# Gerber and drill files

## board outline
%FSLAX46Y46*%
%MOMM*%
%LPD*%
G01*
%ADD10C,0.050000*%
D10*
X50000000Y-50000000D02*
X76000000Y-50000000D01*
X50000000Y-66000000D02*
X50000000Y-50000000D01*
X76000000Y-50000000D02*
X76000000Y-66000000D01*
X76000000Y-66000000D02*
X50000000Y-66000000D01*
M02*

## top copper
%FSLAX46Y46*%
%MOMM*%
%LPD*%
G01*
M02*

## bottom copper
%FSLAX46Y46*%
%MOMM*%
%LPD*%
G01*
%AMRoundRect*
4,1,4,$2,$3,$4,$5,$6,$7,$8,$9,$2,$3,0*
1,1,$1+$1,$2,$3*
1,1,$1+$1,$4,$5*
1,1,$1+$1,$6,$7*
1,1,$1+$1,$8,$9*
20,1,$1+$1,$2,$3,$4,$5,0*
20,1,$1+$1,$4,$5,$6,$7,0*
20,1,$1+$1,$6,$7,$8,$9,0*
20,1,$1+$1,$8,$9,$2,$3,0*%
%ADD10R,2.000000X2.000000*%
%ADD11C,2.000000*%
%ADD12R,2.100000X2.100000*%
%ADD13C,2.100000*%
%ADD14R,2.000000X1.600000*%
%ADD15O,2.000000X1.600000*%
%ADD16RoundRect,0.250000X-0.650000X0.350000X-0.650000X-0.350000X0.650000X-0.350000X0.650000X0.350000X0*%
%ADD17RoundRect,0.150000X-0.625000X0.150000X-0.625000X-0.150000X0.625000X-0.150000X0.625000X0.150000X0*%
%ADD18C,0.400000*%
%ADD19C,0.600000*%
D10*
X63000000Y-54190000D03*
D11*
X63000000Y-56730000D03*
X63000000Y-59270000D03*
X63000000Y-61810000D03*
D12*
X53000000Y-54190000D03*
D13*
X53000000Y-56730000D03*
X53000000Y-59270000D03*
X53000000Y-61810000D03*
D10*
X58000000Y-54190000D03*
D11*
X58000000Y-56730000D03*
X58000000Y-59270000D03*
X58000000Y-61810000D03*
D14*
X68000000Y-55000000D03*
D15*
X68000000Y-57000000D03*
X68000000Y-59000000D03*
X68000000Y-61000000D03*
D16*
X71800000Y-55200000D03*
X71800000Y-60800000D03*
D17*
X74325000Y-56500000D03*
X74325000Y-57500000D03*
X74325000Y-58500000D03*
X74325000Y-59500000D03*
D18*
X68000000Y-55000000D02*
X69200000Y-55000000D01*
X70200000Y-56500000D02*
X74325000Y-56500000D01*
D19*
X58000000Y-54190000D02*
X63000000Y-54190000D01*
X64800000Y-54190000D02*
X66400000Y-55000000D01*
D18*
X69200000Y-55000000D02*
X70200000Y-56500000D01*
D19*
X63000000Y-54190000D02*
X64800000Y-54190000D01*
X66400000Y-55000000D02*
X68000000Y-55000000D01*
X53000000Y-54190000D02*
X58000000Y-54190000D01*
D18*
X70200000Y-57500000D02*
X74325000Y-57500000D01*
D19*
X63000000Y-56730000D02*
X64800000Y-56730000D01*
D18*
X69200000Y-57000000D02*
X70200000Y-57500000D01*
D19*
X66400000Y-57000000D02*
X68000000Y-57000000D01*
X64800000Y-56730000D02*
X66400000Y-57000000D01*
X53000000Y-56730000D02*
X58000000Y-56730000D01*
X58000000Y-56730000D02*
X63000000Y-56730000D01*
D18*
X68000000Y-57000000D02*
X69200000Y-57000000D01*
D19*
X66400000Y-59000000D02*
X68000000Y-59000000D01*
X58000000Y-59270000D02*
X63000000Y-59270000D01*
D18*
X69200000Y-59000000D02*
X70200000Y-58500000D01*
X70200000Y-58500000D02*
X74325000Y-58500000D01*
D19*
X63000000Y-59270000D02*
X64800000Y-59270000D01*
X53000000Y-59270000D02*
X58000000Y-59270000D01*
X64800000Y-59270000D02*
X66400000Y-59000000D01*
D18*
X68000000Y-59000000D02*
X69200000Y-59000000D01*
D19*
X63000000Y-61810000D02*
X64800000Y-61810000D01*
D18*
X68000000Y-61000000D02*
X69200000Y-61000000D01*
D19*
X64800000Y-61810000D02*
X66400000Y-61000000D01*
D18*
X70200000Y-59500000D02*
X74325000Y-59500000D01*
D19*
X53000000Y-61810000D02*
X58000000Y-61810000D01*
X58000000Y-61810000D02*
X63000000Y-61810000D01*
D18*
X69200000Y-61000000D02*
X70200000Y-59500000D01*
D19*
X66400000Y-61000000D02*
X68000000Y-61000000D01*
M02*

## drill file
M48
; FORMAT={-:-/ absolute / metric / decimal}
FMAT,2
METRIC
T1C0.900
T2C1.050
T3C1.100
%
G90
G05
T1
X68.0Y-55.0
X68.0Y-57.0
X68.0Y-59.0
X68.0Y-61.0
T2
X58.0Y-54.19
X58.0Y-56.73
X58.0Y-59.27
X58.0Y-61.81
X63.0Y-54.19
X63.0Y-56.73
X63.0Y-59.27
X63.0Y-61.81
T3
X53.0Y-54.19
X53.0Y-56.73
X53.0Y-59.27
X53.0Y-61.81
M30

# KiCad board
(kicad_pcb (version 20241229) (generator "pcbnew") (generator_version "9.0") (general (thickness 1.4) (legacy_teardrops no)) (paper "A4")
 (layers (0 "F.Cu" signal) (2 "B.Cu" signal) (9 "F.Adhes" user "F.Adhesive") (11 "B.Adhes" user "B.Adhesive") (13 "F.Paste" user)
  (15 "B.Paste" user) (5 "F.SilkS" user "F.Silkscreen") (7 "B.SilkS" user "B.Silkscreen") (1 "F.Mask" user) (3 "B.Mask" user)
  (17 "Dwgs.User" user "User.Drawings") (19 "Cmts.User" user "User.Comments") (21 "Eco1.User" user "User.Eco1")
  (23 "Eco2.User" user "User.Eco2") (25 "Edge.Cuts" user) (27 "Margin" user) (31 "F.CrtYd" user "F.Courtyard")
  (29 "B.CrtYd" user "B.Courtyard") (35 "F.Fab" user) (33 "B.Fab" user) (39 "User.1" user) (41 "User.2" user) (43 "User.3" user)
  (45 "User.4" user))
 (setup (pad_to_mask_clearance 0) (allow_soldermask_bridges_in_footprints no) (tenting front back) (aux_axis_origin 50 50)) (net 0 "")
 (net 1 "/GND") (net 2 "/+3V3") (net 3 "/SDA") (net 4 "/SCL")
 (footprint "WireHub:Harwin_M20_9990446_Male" (layer "F.Cu") (at 63 54.19)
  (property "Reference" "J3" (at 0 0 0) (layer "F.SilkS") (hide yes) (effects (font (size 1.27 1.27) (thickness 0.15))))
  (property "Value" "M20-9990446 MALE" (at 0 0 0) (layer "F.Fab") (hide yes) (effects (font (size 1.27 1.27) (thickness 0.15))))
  (pad "1" thru_hole rect (at 0 0) (size 2 2) (drill 1.05) (layers "*.Cu" "*.Mask") (remove_unused_layers yes) (keep_end_layers no)
   (zone_layer_connections) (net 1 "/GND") (thermal_bridge_angle 45))
  (pad "2" thru_hole circle (at 0 2.54) (size 2 2) (drill 1.05) (layers "*.Cu" "*.Mask") (remove_unused_layers yes) (keep_end_layers no)
   (zone_layer_connections) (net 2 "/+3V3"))
  (pad "3" thru_hole circle (at 0 5.08) (size 2 2) (drill 1.05) (layers "*.Cu" "*.Mask") (remove_unused_layers yes) (keep_end_layers no)
   (zone_layer_connections) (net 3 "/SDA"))
  (pad "4" thru_hole circle (at 0 7.62) (size 2 2) (drill 1.05) (layers "*.Cu" "*.Mask") (remove_unused_layers yes) (keep_end_layers no)
   (zone_layer_connections) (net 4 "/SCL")))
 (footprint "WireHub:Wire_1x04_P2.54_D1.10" (layer "F.Cu") (at 53 54.19)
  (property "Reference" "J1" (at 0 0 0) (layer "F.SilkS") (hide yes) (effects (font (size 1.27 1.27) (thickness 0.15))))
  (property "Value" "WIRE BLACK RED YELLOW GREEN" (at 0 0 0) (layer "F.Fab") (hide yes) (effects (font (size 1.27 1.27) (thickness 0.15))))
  (pad "1" thru_hole rect (at 0 0) (size 2.1 2.1) (drill 1.1) (layers "*.Cu" "*.Mask") (remove_unused_layers yes) (keep_end_layers no)
   (zone_layer_connections) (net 1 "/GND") (thermal_bridge_angle 45))
  (pad "2" thru_hole circle (at 0 2.54) (size 2.1 2.1) (drill 1.1) (layers "*.Cu" "*.Mask") (remove_unused_layers yes) (keep_end_layers no)
   (zone_layer_connections) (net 2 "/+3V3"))
  (pad "3" thru_hole circle (at 0 5.08) (size 2.1 2.1) (drill 1.1) (layers "*.Cu" "*.Mask") (remove_unused_layers yes) (keep_end_layers no)
   (zone_layer_connections) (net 3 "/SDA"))
  (pad "4" thru_hole circle (at 0 7.62) (size 2.1 2.1) (drill 1.1) (layers "*.Cu" "*.Mask") (remove_unused_layers yes) (keep_end_layers no)
   (zone_layer_connections) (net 4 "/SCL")))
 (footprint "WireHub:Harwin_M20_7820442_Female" (layer "F.Cu") (at 58 54.19)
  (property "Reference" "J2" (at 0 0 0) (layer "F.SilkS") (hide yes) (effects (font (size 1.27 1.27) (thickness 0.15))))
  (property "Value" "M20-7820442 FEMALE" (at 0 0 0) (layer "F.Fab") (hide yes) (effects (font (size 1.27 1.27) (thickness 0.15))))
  (pad "1" thru_hole rect (at 0 0) (size 2 2) (drill 1.05) (layers "*.Cu" "*.Mask") (remove_unused_layers yes) (keep_end_layers no)
   (zone_layer_connections) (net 1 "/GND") (thermal_bridge_angle 45))
  (pad "2" thru_hole circle (at 0 2.54) (size 2 2) (drill 1.05) (layers "*.Cu" "*.Mask") (remove_unused_layers yes) (keep_end_layers no)
   (zone_layer_connections) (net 2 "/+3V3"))
  (pad "3" thru_hole circle (at 0 5.08) (size 2 2) (drill 1.05) (layers "*.Cu" "*.Mask") (remove_unused_layers yes) (keep_end_layers no)
   (zone_layer_connections) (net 3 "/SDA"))
  (pad "4" thru_hole circle (at 0 7.62) (size 2 2) (drill 1.05) (layers "*.Cu" "*.Mask") (remove_unused_layers yes) (keep_end_layers no)
   (zone_layer_connections) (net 4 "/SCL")))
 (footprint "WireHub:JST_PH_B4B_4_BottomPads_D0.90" (layer "F.Cu") (at 68 55 -90)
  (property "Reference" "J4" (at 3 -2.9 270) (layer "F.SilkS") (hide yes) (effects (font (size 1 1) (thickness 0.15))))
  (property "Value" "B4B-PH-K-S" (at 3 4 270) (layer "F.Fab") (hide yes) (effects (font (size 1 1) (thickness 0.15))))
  (pad "1" thru_hole rect (at 0 0 270) (size 1.6 2) (drill 0.9) (layers "*.Cu" "*.Mask") (remove_unused_layers yes) (keep_end_layers no)
   (zone_layer_connections) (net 1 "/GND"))
  (pad "2" thru_hole oval (at 2 0 270) (size 1.6 2) (drill 0.9) (layers "*.Cu" "*.Mask") (remove_unused_layers yes) (keep_end_layers no)
   (zone_layer_connections) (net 2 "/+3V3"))
  (pad "3" thru_hole oval (at 4 0 270) (size 1.6 2) (drill 0.9) (layers "*.Cu" "*.Mask") (remove_unused_layers yes) (keep_end_layers no)
   (zone_layer_connections) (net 3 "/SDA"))
  (pad "4" thru_hole oval (at 6 0 270) (size 1.6 2) (drill 0.9) (layers "*.Cu" "*.Mask") (remove_unused_layers yes) (keep_end_layers no)
   (zone_layer_connections) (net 4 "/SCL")))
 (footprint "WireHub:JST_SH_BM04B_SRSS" (layer "B.Cu") (at 73 58 -90)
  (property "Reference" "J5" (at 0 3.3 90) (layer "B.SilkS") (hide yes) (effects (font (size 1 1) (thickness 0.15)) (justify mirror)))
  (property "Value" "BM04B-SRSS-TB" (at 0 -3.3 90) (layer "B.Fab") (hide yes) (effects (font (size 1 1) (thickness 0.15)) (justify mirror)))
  (pad "" smd roundrect (at -2.8 1.2 270) (size 1.2 1.8) (layers "B.Cu" "B.Mask" "B.Paste") (roundrect_rratio 0.208333))
  (pad "" smd roundrect (at 2.8 1.2 270) (size 1.2 1.8) (layers "B.Cu" "B.Mask" "B.Paste") (roundrect_rratio 0.208333))
  (pad "1" smd roundrect (at -1.5 -1.325 270) (size 0.6 1.55) (layers "B.Cu" "B.Mask" "B.Paste") (roundrect_rratio 0.25) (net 1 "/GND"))
  (pad "2" smd roundrect (at -0.5 -1.325 270) (size 0.6 1.55) (layers "B.Cu" "B.Mask" "B.Paste") (roundrect_rratio 0.25) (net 2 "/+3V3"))
  (pad "3" smd roundrect (at 0.5 -1.325 270) (size 0.6 1.55) (layers "B.Cu" "B.Mask" "B.Paste") (roundrect_rratio 0.25) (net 3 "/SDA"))
  (pad "4" smd roundrect (at 1.5 -1.325 270) (size 0.6 1.55) (layers "B.Cu" "B.Mask" "B.Paste") (roundrect_rratio 0.25) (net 4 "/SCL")))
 (gr_line (start 50 50) (end 76 50) (stroke (width 0.05) (type default)) (layer "Edge.Cuts"))
 (gr_line (start 50 66) (end 50 50) (stroke (width 0.05) (type default)) (layer "Edge.Cuts"))
 (gr_line (start 76 50) (end 76 66) (stroke (width 0.05) (type default)) (layer "Edge.Cuts"))
 (gr_line (start 76 66) (end 50 66) (stroke (width 0.05) (type default)) (layer "Edge.Cuts"))
 (segment (start 68 55) (end 69.2 55) (width 0.4) (layer "B.Cu") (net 1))
 (segment (start 70.2 56.5) (end 74.325 56.5) (width 0.4) (layer "B.Cu") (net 1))
 (segment (start 58 54.19) (end 63 54.19) (width 0.6) (layer "B.Cu") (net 1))
 (segment (start 64.8 54.19) (end 66.4 55) (width 0.6) (layer "B.Cu") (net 1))
 (segment (start 69.2 55) (end 70.2 56.5) (width 0.4) (layer "B.Cu") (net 1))
 (segment (start 63 54.19) (end 64.8 54.19) (width 0.6) (layer "B.Cu") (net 1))
 (segment (start 66.4 55) (end 68 55) (width 0.6) (layer "B.Cu") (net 1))
 (segment (start 53 54.19) (end 58 54.19) (width 0.6) (layer "B.Cu") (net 1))
 (segment (start 70.2 57.5) (end 74.325 57.5) (width 0.4) (layer "B.Cu") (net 2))
 (segment (start 63 56.73) (end 64.8 56.73) (width 0.6) (layer "B.Cu") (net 2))
 (segment (start 69.2 57) (end 70.2 57.5) (width 0.4) (layer "B.Cu") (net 2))
 (segment (start 66.4 57) (end 68 57) (width 0.6) (layer "B.Cu") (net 2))
 (segment (start 64.8 56.73) (end 66.4 57) (width 0.6) (layer "B.Cu") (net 2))
 (segment (start 53 56.73) (end 58 56.73) (width 0.6) (layer "B.Cu") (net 2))
 (segment (start 58 56.73) (end 63 56.73) (width 0.6) (layer "B.Cu") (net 2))
 (segment (start 68 57) (end 69.2 57) (width 0.4) (layer "B.Cu") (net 2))
 (segment (start 66.4 59) (end 68 59) (width 0.6) (layer "B.Cu") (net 3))
 (segment (start 58 59.27) (end 63 59.27) (width 0.6) (layer "B.Cu") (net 3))
 (segment (start 69.2 59) (end 70.2 58.5) (width 0.4) (layer "B.Cu") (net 3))
 (segment (start 70.2 58.5) (end 74.325 58.5) (width 0.4) (layer "B.Cu") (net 3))
 (segment (start 63 59.27) (end 64.8 59.27) (width 0.6) (layer "B.Cu") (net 3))
 (segment (start 53 59.27) (end 58 59.27) (width 0.6) (layer "B.Cu") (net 3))
 (segment (start 64.8 59.27) (end 66.4 59) (width 0.6) (layer "B.Cu") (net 3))
 (segment (start 68 59) (end 69.2 59) (width 0.4) (layer "B.Cu") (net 3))
 (segment (start 63 61.81) (end 64.8 61.81) (width 0.6) (layer "B.Cu") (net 4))
 (segment (start 68 61) (end 69.2 61) (width 0.4) (layer "B.Cu") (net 4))
 (segment (start 64.8 61.81) (end 66.4 61) (width 0.6) (layer "B.Cu") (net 4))
 (segment (start 70.2 59.5) (end 74.325 59.5) (width 0.4) (layer "B.Cu") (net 4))
 (segment (start 53 61.81) (end 58 61.81) (width 0.6) (layer "B.Cu") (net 4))
 (segment (start 58 61.81) (end 63 61.81) (width 0.6) (layer "B.Cu") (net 4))
 (segment (start 69.2 61) (end 70.2 59.5) (width 0.4) (layer "B.Cu") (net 4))
 (segment (start 66.4 61) (end 68 61) (width 0.6) (layer "B.Cu") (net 4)))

